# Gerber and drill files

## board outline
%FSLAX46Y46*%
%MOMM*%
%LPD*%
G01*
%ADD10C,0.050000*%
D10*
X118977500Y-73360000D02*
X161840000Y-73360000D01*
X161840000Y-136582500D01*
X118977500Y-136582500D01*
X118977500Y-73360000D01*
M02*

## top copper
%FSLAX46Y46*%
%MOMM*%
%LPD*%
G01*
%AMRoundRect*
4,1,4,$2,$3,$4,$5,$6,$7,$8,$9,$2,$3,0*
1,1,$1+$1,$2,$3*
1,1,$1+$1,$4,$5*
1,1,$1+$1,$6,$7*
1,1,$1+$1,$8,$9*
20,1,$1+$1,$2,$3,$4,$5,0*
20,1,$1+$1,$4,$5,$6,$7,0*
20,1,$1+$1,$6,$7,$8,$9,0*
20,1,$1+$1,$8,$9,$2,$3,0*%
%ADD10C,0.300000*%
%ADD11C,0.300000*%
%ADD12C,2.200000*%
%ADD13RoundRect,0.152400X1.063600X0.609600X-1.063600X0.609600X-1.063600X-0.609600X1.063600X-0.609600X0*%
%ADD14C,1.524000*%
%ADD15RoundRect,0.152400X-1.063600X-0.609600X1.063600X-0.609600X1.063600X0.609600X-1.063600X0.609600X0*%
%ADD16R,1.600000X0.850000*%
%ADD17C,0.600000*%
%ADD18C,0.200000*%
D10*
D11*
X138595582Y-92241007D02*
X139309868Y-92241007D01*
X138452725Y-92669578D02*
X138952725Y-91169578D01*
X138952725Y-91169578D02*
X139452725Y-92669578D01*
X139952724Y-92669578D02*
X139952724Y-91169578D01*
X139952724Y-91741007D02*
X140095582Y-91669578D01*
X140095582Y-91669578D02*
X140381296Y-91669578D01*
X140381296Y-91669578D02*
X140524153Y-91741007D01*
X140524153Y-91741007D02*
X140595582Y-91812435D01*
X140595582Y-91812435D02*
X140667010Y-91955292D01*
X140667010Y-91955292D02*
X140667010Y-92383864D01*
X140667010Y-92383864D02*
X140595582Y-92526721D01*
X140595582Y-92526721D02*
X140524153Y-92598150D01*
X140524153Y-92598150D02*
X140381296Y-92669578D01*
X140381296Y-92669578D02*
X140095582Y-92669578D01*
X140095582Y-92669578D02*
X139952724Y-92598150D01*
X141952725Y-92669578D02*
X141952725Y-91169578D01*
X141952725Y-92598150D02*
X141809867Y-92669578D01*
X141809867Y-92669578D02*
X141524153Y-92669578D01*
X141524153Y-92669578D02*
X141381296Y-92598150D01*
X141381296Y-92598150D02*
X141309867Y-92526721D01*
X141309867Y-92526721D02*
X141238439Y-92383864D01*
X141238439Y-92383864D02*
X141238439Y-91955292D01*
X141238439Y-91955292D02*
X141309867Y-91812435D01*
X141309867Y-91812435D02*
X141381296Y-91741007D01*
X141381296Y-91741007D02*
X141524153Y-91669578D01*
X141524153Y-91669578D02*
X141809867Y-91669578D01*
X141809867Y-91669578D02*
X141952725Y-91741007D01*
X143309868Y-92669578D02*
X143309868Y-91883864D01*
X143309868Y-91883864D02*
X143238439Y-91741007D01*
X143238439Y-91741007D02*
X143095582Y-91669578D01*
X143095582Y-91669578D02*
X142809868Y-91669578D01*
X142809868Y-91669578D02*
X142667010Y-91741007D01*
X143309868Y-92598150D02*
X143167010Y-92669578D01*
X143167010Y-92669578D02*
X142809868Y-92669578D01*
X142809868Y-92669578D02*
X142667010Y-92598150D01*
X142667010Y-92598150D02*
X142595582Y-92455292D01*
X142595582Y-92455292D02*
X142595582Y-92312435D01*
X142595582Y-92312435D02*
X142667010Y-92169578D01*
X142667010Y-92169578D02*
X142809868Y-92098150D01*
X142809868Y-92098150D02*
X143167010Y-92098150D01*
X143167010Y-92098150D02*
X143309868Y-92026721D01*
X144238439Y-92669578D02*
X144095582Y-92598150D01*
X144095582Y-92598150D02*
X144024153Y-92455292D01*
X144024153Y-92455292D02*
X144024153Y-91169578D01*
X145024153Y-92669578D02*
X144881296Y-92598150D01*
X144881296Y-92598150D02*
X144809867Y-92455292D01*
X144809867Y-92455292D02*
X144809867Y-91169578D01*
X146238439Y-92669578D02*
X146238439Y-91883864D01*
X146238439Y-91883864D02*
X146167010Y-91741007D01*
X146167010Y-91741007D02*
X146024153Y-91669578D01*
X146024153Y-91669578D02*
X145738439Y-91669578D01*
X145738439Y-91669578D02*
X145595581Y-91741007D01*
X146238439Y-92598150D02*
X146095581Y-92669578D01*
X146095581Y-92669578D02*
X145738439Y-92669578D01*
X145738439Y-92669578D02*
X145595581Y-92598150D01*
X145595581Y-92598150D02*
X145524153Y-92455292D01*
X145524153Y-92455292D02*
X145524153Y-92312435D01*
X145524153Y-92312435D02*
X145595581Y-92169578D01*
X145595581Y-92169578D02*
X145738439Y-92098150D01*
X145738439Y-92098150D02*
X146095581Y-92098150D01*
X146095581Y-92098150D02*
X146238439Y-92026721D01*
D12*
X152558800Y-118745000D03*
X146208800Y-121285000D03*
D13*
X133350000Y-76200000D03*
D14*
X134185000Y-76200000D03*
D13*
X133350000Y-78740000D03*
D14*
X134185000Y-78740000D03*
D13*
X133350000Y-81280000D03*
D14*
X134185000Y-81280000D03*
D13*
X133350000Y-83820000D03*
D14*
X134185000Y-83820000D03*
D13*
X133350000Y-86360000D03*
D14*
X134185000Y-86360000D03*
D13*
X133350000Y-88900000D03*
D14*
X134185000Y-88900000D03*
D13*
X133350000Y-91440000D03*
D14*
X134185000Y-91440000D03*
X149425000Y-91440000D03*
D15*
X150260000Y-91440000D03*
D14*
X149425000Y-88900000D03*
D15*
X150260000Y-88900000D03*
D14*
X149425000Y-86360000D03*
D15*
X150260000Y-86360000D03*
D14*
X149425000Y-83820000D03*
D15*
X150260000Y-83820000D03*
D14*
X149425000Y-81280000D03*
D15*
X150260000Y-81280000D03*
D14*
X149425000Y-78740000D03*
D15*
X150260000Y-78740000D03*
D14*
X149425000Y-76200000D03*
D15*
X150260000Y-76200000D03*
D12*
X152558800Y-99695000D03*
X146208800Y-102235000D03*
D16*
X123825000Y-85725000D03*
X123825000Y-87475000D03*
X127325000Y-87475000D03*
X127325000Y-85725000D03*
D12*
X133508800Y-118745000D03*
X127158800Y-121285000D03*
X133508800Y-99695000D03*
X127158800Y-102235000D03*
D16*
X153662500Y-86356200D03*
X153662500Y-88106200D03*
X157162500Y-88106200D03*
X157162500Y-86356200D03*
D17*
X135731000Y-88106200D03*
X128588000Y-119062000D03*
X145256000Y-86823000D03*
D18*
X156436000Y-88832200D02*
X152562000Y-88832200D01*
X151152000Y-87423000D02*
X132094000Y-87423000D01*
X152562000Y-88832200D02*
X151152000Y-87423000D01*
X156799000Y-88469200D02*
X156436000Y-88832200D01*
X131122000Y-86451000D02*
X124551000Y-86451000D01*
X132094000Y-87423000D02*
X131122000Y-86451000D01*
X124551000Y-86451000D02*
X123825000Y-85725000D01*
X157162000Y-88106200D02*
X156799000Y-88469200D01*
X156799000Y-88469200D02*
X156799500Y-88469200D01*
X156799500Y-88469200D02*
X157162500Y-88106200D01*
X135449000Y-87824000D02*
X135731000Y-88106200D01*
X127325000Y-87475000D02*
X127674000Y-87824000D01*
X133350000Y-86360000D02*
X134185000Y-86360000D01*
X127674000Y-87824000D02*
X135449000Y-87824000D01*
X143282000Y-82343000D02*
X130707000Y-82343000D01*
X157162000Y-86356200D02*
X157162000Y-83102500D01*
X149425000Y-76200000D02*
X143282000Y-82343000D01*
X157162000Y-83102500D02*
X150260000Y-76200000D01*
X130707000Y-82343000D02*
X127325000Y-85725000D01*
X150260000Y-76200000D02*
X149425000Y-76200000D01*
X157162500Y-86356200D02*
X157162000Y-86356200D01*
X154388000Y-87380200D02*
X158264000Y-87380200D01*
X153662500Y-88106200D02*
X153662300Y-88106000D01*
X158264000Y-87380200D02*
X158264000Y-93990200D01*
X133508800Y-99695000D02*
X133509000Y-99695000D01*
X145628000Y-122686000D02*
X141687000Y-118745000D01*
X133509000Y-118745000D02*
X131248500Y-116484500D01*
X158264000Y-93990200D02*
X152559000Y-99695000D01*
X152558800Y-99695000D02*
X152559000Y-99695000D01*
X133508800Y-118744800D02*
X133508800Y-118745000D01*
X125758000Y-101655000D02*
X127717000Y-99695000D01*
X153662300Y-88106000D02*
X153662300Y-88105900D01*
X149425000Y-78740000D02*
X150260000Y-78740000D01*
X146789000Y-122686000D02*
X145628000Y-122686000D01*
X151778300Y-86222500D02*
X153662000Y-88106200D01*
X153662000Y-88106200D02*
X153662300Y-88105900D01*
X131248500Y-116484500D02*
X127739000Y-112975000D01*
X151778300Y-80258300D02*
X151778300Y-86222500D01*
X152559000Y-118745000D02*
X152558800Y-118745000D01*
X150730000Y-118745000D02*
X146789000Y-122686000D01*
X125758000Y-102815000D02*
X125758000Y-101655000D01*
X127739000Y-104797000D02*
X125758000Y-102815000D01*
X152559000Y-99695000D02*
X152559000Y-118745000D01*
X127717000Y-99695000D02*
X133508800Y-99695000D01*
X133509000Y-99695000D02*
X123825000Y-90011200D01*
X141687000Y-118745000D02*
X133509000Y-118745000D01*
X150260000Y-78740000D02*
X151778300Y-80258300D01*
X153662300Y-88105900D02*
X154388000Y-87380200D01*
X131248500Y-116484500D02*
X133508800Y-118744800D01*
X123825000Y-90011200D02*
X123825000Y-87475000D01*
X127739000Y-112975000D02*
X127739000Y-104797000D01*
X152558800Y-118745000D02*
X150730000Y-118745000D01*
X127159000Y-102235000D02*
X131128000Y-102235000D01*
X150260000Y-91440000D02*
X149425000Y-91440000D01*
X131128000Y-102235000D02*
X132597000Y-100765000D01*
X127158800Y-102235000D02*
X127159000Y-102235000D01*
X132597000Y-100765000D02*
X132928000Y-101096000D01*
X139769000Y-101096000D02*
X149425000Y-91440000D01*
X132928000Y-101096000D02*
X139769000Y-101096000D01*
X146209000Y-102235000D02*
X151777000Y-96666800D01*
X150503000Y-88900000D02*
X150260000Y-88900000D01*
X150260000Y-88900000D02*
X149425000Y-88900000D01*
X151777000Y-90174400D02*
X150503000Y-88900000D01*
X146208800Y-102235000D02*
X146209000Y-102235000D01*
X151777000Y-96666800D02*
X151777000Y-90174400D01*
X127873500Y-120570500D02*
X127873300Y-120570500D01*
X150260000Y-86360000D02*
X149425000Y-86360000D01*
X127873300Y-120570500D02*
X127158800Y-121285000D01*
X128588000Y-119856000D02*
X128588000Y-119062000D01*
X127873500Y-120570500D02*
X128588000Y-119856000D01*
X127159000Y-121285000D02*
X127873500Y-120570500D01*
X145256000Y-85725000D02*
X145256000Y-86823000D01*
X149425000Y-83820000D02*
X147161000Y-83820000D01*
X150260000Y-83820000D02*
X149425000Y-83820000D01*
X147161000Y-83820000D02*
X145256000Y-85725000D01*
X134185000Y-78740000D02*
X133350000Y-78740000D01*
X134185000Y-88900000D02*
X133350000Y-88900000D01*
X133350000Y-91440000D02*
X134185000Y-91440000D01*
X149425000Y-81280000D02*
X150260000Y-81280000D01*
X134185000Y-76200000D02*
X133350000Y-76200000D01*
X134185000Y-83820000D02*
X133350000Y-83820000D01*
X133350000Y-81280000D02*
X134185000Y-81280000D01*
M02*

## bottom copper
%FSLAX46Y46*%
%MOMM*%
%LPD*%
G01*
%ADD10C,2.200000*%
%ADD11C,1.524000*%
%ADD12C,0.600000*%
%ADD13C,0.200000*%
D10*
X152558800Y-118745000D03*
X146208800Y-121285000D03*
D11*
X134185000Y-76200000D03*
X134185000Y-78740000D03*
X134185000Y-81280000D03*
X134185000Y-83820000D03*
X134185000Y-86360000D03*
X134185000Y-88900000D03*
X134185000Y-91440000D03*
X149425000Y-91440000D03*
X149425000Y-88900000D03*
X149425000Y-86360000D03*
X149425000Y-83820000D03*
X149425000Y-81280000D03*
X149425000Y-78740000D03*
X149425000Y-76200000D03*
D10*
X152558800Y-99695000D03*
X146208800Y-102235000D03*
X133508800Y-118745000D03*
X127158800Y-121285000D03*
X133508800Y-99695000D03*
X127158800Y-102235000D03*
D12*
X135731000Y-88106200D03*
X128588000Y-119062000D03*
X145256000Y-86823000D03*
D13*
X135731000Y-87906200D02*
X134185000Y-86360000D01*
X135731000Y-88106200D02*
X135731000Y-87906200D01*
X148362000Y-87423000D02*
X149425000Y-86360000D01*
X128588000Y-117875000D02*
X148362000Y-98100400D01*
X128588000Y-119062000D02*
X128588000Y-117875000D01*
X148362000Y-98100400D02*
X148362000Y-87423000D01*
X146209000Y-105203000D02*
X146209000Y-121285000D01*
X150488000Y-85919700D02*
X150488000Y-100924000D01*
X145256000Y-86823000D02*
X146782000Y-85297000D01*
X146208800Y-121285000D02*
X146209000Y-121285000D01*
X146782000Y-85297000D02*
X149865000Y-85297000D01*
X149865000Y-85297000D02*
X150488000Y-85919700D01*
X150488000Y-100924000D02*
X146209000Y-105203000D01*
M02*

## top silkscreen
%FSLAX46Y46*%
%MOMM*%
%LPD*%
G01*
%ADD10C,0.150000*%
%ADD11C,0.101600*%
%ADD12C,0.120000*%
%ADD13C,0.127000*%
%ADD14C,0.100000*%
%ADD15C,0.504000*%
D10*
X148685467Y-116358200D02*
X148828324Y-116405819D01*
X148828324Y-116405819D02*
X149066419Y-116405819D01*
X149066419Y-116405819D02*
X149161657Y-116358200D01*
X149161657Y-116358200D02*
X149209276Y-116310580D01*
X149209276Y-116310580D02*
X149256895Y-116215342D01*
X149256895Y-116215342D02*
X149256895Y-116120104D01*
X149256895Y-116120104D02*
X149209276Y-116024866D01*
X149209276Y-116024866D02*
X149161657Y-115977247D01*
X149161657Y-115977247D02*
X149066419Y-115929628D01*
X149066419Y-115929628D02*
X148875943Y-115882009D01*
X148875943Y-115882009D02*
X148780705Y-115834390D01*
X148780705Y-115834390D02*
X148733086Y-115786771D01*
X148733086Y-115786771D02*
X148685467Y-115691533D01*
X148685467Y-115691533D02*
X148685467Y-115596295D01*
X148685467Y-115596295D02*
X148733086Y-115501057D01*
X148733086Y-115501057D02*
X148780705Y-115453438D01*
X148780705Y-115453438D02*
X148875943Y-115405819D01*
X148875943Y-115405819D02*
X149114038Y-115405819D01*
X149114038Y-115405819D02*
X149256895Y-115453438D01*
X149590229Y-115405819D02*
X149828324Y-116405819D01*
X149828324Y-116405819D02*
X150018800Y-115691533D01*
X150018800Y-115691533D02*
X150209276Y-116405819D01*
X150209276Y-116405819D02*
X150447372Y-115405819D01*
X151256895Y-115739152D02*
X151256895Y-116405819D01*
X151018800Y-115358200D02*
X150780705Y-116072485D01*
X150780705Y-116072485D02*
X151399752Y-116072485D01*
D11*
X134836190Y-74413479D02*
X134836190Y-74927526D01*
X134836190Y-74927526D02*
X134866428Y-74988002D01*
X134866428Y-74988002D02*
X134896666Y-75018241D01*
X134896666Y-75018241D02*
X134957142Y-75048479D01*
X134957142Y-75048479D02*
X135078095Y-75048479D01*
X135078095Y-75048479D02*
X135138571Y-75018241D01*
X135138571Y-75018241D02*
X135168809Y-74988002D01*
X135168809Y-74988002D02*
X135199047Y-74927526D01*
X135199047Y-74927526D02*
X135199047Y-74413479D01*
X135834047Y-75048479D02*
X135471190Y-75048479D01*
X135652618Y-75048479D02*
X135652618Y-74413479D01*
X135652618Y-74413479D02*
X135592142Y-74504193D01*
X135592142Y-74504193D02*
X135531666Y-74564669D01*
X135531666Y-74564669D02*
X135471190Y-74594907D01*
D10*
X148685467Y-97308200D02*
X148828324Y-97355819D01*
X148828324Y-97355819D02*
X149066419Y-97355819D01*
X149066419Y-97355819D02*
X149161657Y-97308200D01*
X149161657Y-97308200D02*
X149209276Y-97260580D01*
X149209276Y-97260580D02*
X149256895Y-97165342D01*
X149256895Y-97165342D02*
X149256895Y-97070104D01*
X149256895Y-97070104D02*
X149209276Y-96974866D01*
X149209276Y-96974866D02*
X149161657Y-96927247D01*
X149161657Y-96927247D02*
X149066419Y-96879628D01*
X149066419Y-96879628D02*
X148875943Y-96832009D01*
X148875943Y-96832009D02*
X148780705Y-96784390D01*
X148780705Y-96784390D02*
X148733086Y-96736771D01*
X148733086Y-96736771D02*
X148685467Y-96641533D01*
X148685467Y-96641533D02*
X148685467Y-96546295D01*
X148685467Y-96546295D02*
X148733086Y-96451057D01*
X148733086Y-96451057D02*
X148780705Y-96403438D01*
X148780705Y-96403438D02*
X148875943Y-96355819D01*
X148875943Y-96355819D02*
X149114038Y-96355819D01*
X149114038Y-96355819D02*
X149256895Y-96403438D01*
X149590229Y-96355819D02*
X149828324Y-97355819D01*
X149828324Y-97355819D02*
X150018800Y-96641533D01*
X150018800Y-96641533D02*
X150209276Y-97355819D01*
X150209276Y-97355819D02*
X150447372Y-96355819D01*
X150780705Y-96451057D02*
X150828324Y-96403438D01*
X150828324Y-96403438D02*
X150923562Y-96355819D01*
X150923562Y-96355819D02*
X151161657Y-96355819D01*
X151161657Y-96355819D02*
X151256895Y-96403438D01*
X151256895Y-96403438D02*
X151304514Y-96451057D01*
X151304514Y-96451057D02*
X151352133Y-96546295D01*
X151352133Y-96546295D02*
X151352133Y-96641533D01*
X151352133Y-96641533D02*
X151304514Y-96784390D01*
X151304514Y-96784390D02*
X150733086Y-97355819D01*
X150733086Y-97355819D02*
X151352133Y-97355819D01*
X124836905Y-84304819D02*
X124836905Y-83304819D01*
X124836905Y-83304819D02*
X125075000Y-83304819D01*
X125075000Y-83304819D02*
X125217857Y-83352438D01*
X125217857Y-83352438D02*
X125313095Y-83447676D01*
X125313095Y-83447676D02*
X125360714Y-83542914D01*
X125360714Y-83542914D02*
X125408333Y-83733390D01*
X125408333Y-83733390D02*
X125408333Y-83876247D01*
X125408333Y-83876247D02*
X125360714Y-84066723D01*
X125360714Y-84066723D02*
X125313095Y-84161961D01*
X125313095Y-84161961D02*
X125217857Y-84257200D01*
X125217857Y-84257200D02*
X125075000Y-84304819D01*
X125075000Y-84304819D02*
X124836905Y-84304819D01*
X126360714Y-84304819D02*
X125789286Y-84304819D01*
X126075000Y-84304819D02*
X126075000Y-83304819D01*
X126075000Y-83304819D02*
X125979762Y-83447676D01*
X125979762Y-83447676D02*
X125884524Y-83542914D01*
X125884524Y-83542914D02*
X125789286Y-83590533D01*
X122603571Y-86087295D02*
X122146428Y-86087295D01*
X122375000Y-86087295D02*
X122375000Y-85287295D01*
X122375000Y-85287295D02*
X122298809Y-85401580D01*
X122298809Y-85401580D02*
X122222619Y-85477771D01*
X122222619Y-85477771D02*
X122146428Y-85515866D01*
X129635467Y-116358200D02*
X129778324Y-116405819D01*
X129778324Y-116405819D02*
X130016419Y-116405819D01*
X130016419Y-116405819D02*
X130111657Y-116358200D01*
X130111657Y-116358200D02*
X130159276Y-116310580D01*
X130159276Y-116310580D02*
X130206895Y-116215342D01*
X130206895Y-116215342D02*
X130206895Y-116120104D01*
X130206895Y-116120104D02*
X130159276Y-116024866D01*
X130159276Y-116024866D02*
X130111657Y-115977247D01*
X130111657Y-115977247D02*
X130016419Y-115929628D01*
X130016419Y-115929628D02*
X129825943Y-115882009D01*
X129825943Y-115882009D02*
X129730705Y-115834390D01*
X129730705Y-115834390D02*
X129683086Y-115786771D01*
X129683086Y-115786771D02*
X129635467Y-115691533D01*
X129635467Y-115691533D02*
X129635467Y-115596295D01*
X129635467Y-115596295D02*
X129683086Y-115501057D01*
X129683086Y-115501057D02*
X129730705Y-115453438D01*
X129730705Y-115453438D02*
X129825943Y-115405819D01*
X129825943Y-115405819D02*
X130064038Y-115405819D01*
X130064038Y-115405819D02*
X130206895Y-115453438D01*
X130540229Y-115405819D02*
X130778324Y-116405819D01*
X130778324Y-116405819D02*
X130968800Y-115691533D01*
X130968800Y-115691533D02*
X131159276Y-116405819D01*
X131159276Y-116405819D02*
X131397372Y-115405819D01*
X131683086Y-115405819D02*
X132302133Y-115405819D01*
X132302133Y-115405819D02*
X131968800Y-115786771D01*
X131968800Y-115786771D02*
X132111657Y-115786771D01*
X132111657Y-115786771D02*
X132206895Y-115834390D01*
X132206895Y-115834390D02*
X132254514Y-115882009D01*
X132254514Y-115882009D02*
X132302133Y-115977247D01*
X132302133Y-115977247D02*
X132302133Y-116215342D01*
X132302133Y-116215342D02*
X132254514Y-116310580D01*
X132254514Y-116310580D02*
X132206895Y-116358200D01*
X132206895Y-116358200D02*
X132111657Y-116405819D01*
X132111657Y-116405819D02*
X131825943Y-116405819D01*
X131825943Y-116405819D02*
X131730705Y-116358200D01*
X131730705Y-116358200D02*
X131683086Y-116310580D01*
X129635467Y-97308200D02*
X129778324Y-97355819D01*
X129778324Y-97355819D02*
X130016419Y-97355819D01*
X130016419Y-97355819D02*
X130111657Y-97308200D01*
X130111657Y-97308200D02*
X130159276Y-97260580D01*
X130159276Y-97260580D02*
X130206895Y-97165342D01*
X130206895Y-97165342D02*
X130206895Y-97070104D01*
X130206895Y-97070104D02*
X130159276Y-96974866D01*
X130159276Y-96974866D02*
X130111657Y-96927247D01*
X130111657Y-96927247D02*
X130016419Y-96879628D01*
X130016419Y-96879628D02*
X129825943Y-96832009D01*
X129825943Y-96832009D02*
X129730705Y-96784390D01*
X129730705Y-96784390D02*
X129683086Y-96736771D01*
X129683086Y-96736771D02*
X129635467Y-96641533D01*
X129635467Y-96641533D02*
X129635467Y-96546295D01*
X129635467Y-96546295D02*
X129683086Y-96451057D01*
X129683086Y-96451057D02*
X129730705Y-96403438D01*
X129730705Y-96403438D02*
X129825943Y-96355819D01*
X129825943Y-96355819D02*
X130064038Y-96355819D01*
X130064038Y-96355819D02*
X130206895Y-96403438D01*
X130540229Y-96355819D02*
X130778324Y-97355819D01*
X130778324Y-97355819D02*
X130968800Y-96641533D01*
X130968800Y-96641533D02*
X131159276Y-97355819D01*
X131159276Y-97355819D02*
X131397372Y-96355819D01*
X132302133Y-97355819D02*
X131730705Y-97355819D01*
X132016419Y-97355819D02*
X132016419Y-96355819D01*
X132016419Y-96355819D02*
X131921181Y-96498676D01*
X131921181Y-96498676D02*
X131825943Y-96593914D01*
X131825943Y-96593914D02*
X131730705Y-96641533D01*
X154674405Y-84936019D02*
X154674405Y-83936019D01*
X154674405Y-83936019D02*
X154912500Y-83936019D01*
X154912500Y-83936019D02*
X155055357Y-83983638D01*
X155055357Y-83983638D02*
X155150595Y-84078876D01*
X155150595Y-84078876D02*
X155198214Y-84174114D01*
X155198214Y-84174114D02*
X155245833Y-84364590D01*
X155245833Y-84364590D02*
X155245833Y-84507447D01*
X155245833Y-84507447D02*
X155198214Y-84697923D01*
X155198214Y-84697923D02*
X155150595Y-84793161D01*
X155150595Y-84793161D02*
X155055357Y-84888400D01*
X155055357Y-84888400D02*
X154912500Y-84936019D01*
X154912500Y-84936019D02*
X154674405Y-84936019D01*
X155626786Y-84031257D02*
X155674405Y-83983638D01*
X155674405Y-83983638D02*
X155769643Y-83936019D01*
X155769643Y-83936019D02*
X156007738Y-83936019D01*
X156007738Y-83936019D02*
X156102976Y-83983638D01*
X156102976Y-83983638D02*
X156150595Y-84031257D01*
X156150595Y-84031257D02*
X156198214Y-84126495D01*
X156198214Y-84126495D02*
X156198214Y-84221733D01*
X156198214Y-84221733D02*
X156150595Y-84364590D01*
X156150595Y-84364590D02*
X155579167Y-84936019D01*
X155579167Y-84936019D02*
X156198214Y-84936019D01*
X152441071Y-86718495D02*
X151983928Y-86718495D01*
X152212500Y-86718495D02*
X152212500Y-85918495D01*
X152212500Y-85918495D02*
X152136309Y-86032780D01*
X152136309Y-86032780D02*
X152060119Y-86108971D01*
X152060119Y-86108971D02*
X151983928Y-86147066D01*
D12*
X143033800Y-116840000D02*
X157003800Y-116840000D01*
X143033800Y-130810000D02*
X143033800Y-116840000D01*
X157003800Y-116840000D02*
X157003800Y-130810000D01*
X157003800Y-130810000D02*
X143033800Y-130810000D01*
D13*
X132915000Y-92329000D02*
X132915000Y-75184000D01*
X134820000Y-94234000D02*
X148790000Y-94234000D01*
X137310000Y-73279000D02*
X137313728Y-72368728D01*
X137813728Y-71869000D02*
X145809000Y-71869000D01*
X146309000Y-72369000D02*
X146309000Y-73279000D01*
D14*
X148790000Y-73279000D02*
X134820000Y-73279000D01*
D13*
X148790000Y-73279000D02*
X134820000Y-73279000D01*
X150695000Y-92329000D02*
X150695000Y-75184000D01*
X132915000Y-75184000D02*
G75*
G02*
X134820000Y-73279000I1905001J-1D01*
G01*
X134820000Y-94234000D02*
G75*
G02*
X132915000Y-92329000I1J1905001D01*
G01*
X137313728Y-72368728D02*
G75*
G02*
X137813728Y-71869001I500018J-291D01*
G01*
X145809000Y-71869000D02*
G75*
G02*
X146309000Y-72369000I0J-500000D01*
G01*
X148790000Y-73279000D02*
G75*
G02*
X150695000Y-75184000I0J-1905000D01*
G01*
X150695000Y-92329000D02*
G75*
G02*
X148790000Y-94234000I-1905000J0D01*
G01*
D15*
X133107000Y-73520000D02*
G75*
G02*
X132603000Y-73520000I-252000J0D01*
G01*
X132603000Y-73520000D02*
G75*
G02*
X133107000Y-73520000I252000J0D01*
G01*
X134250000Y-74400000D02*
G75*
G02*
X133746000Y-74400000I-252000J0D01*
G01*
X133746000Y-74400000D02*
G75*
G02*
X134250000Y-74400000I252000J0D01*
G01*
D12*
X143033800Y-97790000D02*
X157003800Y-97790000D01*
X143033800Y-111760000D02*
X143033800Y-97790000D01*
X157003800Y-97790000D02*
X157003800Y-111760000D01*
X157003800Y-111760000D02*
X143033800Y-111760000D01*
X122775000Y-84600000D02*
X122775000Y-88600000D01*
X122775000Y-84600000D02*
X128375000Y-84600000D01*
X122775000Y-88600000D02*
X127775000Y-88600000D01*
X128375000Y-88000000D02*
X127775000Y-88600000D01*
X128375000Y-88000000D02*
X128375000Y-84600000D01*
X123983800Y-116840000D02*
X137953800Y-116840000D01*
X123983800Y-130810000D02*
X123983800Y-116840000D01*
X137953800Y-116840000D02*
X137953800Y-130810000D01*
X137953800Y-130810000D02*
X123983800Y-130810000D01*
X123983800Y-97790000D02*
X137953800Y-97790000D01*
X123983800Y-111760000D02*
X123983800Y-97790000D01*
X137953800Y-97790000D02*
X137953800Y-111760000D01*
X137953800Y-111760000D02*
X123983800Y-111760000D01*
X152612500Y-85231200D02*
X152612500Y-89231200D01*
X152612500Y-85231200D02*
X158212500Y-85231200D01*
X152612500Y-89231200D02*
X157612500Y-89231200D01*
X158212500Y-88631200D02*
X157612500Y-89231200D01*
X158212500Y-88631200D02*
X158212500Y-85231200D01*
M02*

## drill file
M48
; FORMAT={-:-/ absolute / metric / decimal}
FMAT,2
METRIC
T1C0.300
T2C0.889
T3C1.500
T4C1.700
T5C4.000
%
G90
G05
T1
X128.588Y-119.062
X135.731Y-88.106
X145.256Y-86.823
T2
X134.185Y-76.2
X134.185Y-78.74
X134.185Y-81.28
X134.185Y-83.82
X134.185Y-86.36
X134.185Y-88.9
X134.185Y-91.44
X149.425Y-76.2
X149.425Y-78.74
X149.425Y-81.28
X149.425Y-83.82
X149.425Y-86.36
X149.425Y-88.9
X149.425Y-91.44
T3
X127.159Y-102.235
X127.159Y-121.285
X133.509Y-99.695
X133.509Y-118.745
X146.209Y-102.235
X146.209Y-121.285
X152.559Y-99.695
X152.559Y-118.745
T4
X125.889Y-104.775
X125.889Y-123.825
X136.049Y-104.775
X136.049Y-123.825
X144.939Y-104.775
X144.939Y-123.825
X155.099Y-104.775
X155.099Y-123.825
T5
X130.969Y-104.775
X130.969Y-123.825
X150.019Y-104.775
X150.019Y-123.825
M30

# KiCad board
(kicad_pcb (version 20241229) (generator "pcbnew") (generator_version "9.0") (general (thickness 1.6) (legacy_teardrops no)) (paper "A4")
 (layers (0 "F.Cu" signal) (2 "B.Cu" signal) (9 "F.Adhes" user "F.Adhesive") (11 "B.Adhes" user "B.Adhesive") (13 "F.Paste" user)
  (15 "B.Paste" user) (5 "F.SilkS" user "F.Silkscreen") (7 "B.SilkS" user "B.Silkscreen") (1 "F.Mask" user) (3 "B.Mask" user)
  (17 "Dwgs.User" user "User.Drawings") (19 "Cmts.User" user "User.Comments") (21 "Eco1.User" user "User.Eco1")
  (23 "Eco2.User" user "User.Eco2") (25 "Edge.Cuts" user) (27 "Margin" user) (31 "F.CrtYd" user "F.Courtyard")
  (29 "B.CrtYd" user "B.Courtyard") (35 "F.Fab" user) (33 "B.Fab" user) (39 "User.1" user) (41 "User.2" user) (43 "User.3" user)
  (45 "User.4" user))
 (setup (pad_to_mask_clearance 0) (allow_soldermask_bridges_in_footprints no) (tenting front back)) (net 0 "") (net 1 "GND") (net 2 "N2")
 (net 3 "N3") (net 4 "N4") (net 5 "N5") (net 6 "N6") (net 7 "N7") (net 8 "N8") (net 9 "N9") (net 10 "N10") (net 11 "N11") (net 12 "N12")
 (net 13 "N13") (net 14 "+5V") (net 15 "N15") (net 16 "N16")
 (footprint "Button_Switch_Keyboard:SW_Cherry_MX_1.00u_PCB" (layer "F.Cu") (at 152.5588 118.745)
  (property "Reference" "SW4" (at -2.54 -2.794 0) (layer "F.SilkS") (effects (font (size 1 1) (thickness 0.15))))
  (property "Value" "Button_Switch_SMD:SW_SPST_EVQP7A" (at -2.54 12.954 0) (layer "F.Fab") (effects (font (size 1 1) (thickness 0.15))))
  (fp_line (start -9.525 -1.905) (end 4.445 -1.905) (stroke (width 0.12) (type solid)) (layer "F.SilkS"))
  (fp_line (start -9.525 12.065) (end -9.525 -1.905) (stroke (width 0.12) (type solid)) (layer "F.SilkS"))
  (fp_line (start 4.445 -1.905) (end 4.445 12.065) (stroke (width 0.12) (type solid)) (layer "F.SilkS"))
  (fp_line (start 4.445 12.065) (end -9.525 12.065) (stroke (width 0.12) (type solid)) (layer "F.SilkS"))
  (pad "" np_thru_hole circle (at -7.62 5.08) (size 1.7 1.7) (drill 1.7) (layers "*.Cu" "*.Mask"))
  (pad "" np_thru_hole circle (at -2.54 5.08) (size 4 4) (drill 4) (layers "*.Cu" "*.Mask"))
  (pad "" np_thru_hole circle (at 2.54 5.08) (size 1.7 1.7) (drill 1.7) (layers "*.Cu" "*.Mask"))
  (pad "1" thru_hole circle (at 0 0) (size 2.2 2.2) (drill 1.5) (layers "*.Cu" "*.Mask") (remove_unused_layers no) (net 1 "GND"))
  (pad "2" thru_hole circle (at -6.35 2.54) (size 2.2 2.2) (drill 1.5) (layers "*.Cu" "*.Mask") (remove_unused_layers no) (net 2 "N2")))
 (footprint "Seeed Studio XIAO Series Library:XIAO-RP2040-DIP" (layer "F.Cu") (at 141.805 83.82)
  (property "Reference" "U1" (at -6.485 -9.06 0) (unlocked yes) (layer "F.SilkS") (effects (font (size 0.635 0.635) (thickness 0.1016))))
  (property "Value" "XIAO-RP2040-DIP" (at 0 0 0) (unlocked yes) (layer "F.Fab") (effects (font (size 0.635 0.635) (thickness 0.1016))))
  (fp_line (start -8.89 8.509) (end -8.89 -8.636) (stroke (width 0.127) (type solid)) (layer "F.SilkS"))
  (fp_line (start -6.985 10.414) (end 6.985 10.414) (stroke (width 0.127) (type solid)) (layer "F.SilkS"))
  (fp_line (start -4.495 -10.541) (end -4.491272 -11.451272) (stroke (width 0.127) (type solid)) (layer "F.SilkS"))
  (fp_line (start -3.991272 -11.951) (end 4.004 -11.951) (stroke (width 0.127) (type solid)) (layer "F.SilkS"))
  (fp_line (start 4.504 -11.451) (end 4.504 -10.541) (stroke (width 0.127) (type solid)) (layer "F.SilkS"))
  (fp_line (start 6.985 -10.541) (end -6.985 -10.541) (stroke (width 0.1) (type solid)) (layer "F.SilkS"))
  (fp_line (start 6.985 -10.541) (end -6.985 -10.541) (stroke (width 0.127) (type solid)) (layer "F.SilkS"))
  (fp_line (start 8.89 8.509) (end 8.89 -8.636) (stroke (width 0.127) (type solid)) (layer "F.SilkS"))
  (fp_arc (start -8.89 -8.636) (mid -8.332038 -9.983038) (end -6.985 -10.541) (stroke (width 0.127) (type solid)) (layer "F.SilkS"))
  (fp_arc (start -6.985 10.414) (mid -8.332038 9.856038) (end -8.89 8.509) (stroke (width 0.127) (type solid)) (layer "F.SilkS"))
  (fp_arc (start -4.491272 -11.451272) (mid -4.344728 -11.80464) (end -3.991272 -11.951) (stroke (width 0.127) (type default))
   (layer "F.SilkS"))
  (fp_arc (start 4.004 -11.951) (mid 4.357553 -11.804553) (end 4.504 -11.451) (stroke (width 0.127) (type default)) (layer "F.SilkS"))
  (fp_arc (start 6.985 -10.541) (mid 8.332038 -9.983038) (end 8.89 -8.636) (stroke (width 0.127) (type solid)) (layer "F.SilkS"))
  (fp_arc (start 8.89 8.509) (mid 8.332038 9.856038) (end 6.985 10.414) (stroke (width 0.127) (type solid)) (layer "F.SilkS"))
  (fp_circle (center -8.95 -10.3) (end -8.95 -10.554) (stroke (width 0.5) (type solid)) (fill yes) (layer "F.SilkS"))
  (fp_circle (center -7.807 -9.42) (end -7.807 -9.674) (stroke (width 0.5) (type solid)) (fill yes) (layer "F.SilkS"))
  (pad "1" smd roundrect (at -8.455 -7.62 180) (size 2.432 1.524) (layers "F.Cu" "F.Mask") (roundrect_rratio 0.1) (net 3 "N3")
   (thermal_bridge_angle 45))
  (pad "1" thru_hole circle (at -7.62 -7.62 180) (size 1.524 1.524) (drill 0.889) (layers "*.Cu" "*.Mask") (remove_unused_layers no)
   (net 3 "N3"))
  (pad "2" smd roundrect (at -8.455 -5.08 180) (size 2.432 1.524) (layers "F.Cu" "F.Mask") (roundrect_rratio 0.1) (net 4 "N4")
   (thermal_bridge_angle 45))
  (pad "2" thru_hole circle (at -7.62 -5.08 180) (size 1.524 1.524) (drill 0.889) (layers "*.Cu" "*.Mask") (remove_unused_layers no)
   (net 4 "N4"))
  (pad "3" smd roundrect (at -8.455 -2.54 180) (size 2.432 1.524) (layers "F.Cu" "F.Mask") (roundrect_rratio 0.1) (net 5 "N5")
   (thermal_bridge_angle 45))
  (pad "3" thru_hole circle (at -7.62 -2.54 180) (size 1.524 1.524) (drill 0.889) (layers "*.Cu" "*.Mask") (remove_unused_layers no)
   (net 5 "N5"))
  (pad "4" smd roundrect (at -8.455 0 180) (size 2.432 1.524) (layers "F.Cu" "F.Mask") (roundrect_rratio 0.1) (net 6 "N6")
   (thermal_bridge_angle 45))
  (pad "4" thru_hole circle (at -7.62 0 180) (size 1.524 1.524) (drill 0.889) (layers "*.Cu" "*.Mask") (remove_unused_layers no)
   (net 6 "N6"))
  (pad "5" smd roundrect (at -8.455 2.54 180) (size 2.432 1.524) (layers "F.Cu" "F.Mask") (roundrect_rratio 0.1) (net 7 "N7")
   (thermal_bridge_angle 45))
  (pad "5" thru_hole circle (at -7.62 2.54 180) (size 1.524 1.524) (drill 0.889) (layers "*.Cu" "*.Mask") (remove_unused_layers no)
   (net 7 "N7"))
  (pad "6" smd roundrect (at -8.455 5.08 180) (size 2.432 1.524) (layers "F.Cu" "F.Mask") (roundrect_rratio 0.1) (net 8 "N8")
   (thermal_bridge_angle 45))
  (pad "6" thru_hole circle (at -7.62 5.08 180) (size 1.524 1.524) (drill 0.889) (layers "*.Cu" "*.Mask") (remove_unused_layers no)
   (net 8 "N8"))
  (pad "7" smd roundrect (at -8.455 7.62 180) (size 2.432 1.524) (layers "F.Cu" "F.Mask") (roundrect_rratio 0.1) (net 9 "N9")
   (thermal_bridge_angle 45))
  (pad "7" thru_hole circle (at -7.62 7.62 180) (size 1.524 1.524) (drill 0.889) (layers "*.Cu" "*.Mask") (remove_unused_layers no)
   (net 9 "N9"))
  (pad "8" thru_hole circle (at 7.62 7.62) (size 1.524 1.524) (drill 0.889) (layers "*.Cu" "*.Mask") (remove_unused_layers no)
   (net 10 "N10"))
  (pad "8" smd roundrect (at 8.455 7.62) (size 2.432 1.524) (layers "F.Cu" "F.Mask") (roundrect_rratio 0.1) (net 10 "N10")
   (thermal_bridge_angle 45))
  (pad "9" thru_hole circle (at 7.62 5.08) (size 1.524 1.524) (drill 0.889) (layers "*.Cu" "*.Mask") (remove_unused_layers no)
   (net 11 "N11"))
  (pad "9" smd roundrect (at 8.455 5.08) (size 2.432 1.524) (layers "F.Cu" "F.Mask") (roundrect_rratio 0.1) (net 11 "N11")
   (thermal_bridge_angle 45))
  (pad "10" thru_hole circle (at 7.62 2.54) (size 1.524 1.524) (drill 0.889) (layers "*.Cu" "*.Mask") (remove_unused_layers no)
   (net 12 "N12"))
  (pad "10" smd roundrect (at 8.455 2.54) (size 2.432 1.524) (layers "F.Cu" "F.Mask") (roundrect_rratio 0.1) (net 12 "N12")
   (thermal_bridge_angle 45))
  (pad "11" thru_hole circle (at 7.62 0) (size 1.524 1.524) (drill 0.889) (layers "*.Cu" "*.Mask") (remove_unused_layers no) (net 2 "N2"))
  (pad "11" smd roundrect (at 8.455 0) (size 2.432 1.524) (layers "F.Cu" "F.Mask") (roundrect_rratio 0.1) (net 2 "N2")
   (thermal_bridge_angle 45))
  (pad "12" thru_hole circle (at 7.62 -2.54) (size 1.524 1.524) (drill 0.889) (layers "*.Cu" "*.Mask") (remove_unused_layers no)
   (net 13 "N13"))
  (pad "12" smd roundrect (at 8.455 -2.54) (size 2.432 1.524) (layers "F.Cu" "F.Mask") (roundrect_rratio 0.1) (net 13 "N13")
   (thermal_bridge_angle 45))
  (pad "13" thru_hole circle (at 7.62 -5.08) (size 1.524 1.524) (drill 0.889) (layers "*.Cu" "*.Mask") (remove_unused_layers no)
   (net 1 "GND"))
  (pad "13" smd roundrect (at 8.455 -5.08) (size 2.432 1.524) (layers "F.Cu" "F.Mask") (roundrect_rratio 0.1) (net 1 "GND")
   (thermal_bridge_angle 45))
  (pad "14" thru_hole circle (at 7.62 -7.62) (size 1.524 1.524) (drill 0.889) (layers "*.Cu" "*.Mask") (remove_unused_layers no)
   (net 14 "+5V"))
  (pad "14" smd roundrect (at 8.455 -7.62) (size 2.432 1.524) (layers "F.Cu" "F.Mask") (roundrect_rratio 0.1) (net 14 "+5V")
   (thermal_bridge_angle 45)))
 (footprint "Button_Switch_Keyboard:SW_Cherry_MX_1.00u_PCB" (layer "F.Cu") (at 152.5588 99.695)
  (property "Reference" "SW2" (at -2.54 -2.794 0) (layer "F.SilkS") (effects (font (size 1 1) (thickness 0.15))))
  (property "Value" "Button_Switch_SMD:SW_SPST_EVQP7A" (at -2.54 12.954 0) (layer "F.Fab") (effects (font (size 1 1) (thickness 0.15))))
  (fp_line (start -9.525 -1.905) (end 4.445 -1.905) (stroke (width 0.12) (type solid)) (layer "F.SilkS"))
  (fp_line (start -9.525 12.065) (end -9.525 -1.905) (stroke (width 0.12) (type solid)) (layer "F.SilkS"))
  (fp_line (start 4.445 -1.905) (end 4.445 12.065) (stroke (width 0.12) (type solid)) (layer "F.SilkS"))
  (fp_line (start 4.445 12.065) (end -9.525 12.065) (stroke (width 0.12) (type solid)) (layer "F.SilkS"))
  (pad "" np_thru_hole circle (at -7.62 5.08) (size 1.7 1.7) (drill 1.7) (layers "*.Cu" "*.Mask"))
  (pad "" np_thru_hole circle (at -2.54 5.08) (size 4 4) (drill 4) (layers "*.Cu" "*.Mask"))
  (pad "" np_thru_hole circle (at 2.54 5.08) (size 1.7 1.7) (drill 1.7) (layers "*.Cu" "*.Mask"))
  (pad "1" thru_hole circle (at 0 0) (size 2.2 2.2) (drill 1.5) (layers "*.Cu" "*.Mask") (remove_unused_layers no) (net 1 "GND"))
  (pad "2" thru_hole circle (at -6.35 2.54) (size 2.2 2.2) (drill 1.5) (layers "*.Cu" "*.Mask") (remove_unused_layers no) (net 11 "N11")))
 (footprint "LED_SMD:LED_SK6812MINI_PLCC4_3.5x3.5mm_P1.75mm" (layer "F.Cu") (at 125.575 86.6)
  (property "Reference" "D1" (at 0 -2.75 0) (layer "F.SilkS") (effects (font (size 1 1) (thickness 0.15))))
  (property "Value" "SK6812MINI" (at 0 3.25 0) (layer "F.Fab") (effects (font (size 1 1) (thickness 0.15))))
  (fp_line (start -2.8 -2) (end -2.8 2) (stroke (width 0.12) (type default)) (layer "F.SilkS"))
  (fp_line (start -2.8 -2) (end 2.8 -2) (stroke (width 0.12) (type solid)) (layer "F.SilkS"))
  (fp_line (start -2.8 2) (end 2.2 2) (stroke (width 0.12) (type solid)) (layer "F.SilkS"))
  (fp_line (start 2.8 1.4) (end 2.2 2) (stroke (width 0.12) (type default)) (layer "F.SilkS"))
  (fp_line (start 2.8 1.4) (end 2.8 -2) (stroke (width 0.12) (type solid)) (layer "F.SilkS"))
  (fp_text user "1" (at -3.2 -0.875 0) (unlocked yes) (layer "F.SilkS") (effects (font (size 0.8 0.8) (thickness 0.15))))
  (pad "1" smd rect (at -1.75 -0.875) (size 1.6 0.85) (layers "F.Cu" "F.Mask" "F.Paste") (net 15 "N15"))
  (pad "2" smd rect (at -1.75 0.875) (size 1.6 0.85) (layers "F.Cu" "F.Mask" "F.Paste") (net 1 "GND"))
  (pad "3" smd rect (at 1.75 0.875) (size 1.6 0.85) (layers "F.Cu" "F.Mask" "F.Paste") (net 7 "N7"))
  (pad "4" smd rect (at 1.75 -0.875) (size 1.6 0.85) (layers "F.Cu" "F.Mask" "F.Paste") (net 14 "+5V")))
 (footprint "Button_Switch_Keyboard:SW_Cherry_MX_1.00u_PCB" (layer "F.Cu") (at 133.5088 118.745)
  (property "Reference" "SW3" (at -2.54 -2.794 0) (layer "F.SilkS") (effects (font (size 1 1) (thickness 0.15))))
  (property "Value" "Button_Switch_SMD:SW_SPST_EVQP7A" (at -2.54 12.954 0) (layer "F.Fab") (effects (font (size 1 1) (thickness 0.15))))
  (fp_line (start -9.525 -1.905) (end 4.445 -1.905) (stroke (width 0.12) (type solid)) (layer "F.SilkS"))
  (fp_line (start -9.525 12.065) (end -9.525 -1.905) (stroke (width 0.12) (type solid)) (layer "F.SilkS"))
  (fp_line (start 4.445 -1.905) (end 4.445 12.065) (stroke (width 0.12) (type solid)) (layer "F.SilkS"))
  (fp_line (start 4.445 12.065) (end -9.525 12.065) (stroke (width 0.12) (type solid)) (layer "F.SilkS"))
  (pad "" np_thru_hole circle (at -7.62 5.08) (size 1.7 1.7) (drill 1.7) (layers "*.Cu" "*.Mask"))
  (pad "" np_thru_hole circle (at -2.54 5.08) (size 4 4) (drill 4) (layers "*.Cu" "*.Mask"))
  (pad "" np_thru_hole circle (at 2.54 5.08) (size 1.7 1.7) (drill 1.7) (layers "*.Cu" "*.Mask"))
  (pad "1" thru_hole circle (at 0 0) (size 2.2 2.2) (drill 1.5) (layers "*.Cu" "*.Mask") (remove_unused_layers no) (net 1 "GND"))
  (pad "2" thru_hole circle (at -6.35 2.54) (size 2.2 2.2) (drill 1.5) (layers "*.Cu" "*.Mask") (remove_unused_layers no) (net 12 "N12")))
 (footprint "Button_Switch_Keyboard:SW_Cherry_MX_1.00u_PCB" (layer "F.Cu") (at 133.5088 99.695)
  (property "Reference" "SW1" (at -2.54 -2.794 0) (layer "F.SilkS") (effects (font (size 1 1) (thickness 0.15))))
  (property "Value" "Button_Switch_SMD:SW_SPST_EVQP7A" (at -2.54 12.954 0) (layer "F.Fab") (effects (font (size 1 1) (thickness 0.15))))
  (fp_line (start -9.525 -1.905) (end 4.445 -1.905) (stroke (width 0.12) (type solid)) (layer "F.SilkS"))
  (fp_line (start -9.525 12.065) (end -9.525 -1.905) (stroke (width 0.12) (type solid)) (layer "F.SilkS"))
  (fp_line (start 4.445 -1.905) (end 4.445 12.065) (stroke (width 0.12) (type solid)) (layer "F.SilkS"))
  (fp_line (start 4.445 12.065) (end -9.525 12.065) (stroke (width 0.12) (type solid)) (layer "F.SilkS"))
  (pad "" np_thru_hole circle (at -7.62 5.08) (size 1.7 1.7) (drill 1.7) (layers "*.Cu" "*.Mask"))
  (pad "" np_thru_hole circle (at -2.54 5.08) (size 4 4) (drill 4) (layers "*.Cu" "*.Mask"))
  (pad "" np_thru_hole circle (at 2.54 5.08) (size 1.7 1.7) (drill 1.7) (layers "*.Cu" "*.Mask"))
  (pad "1" thru_hole circle (at 0 0) (size 2.2 2.2) (drill 1.5) (layers "*.Cu" "*.Mask") (remove_unused_layers no) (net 1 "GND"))
  (pad "2" thru_hole circle (at -6.35 2.54) (size 2.2 2.2) (drill 1.5) (layers "*.Cu" "*.Mask") (remove_unused_layers no) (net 10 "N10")))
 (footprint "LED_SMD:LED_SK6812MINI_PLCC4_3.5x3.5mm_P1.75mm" (layer "F.Cu") (at 155.4125 87.2312)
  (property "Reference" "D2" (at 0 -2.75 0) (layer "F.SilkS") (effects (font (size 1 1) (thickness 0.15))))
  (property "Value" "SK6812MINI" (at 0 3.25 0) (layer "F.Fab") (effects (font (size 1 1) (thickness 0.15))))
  (fp_line (start -2.8 -2) (end -2.8 2) (stroke (width 0.12) (type default)) (layer "F.SilkS"))
  (fp_line (start -2.8 -2) (end 2.8 -2) (stroke (width 0.12) (type solid)) (layer "F.SilkS"))
  (fp_line (start -2.8 2) (end 2.2 2) (stroke (width 0.12) (type solid)) (layer "F.SilkS"))
  (fp_line (start 2.8 1.4) (end 2.2 2) (stroke (width 0.12) (type default)) (layer "F.SilkS"))
  (fp_line (start 2.8 1.4) (end 2.8 -2) (stroke (width 0.12) (type solid)) (layer "F.SilkS"))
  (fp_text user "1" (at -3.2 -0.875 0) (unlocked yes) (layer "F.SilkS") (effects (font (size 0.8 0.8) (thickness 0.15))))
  (pad "1" smd rect (at -1.75 -0.875) (size 1.6 0.85) (layers "F.Cu" "F.Mask" "F.Paste") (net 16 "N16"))
  (pad "2" smd rect (at -1.75 0.875) (size 1.6 0.85) (layers "F.Cu" "F.Mask" "F.Paste") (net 1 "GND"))
  (pad "3" smd rect (at 1.75 0.875) (size 1.6 0.85) (layers "F.Cu" "F.Mask" "F.Paste") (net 15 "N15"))
  (pad "4" smd rect (at 1.75 -0.875) (size 1.6 0.85) (layers "F.Cu" "F.Mask" "F.Paste") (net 14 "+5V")))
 (gr_rect (start 118.9775 73.36) (end 161.84 136.5825) (stroke (width 0.05) (type solid)) (fill no) (layer "Edge.Cuts"))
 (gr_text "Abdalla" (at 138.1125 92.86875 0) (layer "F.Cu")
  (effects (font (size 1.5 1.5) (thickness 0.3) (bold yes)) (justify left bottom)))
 (segment (start 156.436 88.8322) (end 152.562 88.8322) (width 0.2) (layer "F.Cu") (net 15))
 (segment (start 151.152 87.423) (end 132.094 87.423) (width 0.2) (layer "F.Cu") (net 15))
 (segment (start 152.562 88.8322) (end 151.152 87.423) (width 0.2) (layer "F.Cu") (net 15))
 (segment (start 156.799 88.4692) (end 156.436 88.8322) (width 0.2) (layer "F.Cu") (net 15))
 (segment (start 131.122 86.451) (end 124.551 86.451) (width 0.2) (layer "F.Cu") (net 15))
 (segment (start 132.094 87.423) (end 131.122 86.451) (width 0.2) (layer "F.Cu") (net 15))
 (segment (start 124.551 86.451) (end 123.825 85.725) (width 0.2) (layer "F.Cu") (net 15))
 (segment (start 157.162 88.1062) (end 156.799 88.4692) (width 0.2) (layer "F.Cu") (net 15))
 (segment (start 156.799 88.4692) (end 156.7995 88.4692) (width 0.2) (layer "F.Cu") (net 15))
 (segment (start 156.7995 88.4692) (end 157.1625 88.1062) (width 0.2) (layer "F.Cu") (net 15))
 (segment (start 135.449 87.824) (end 135.731 88.1062) (width 0.2) (layer "F.Cu") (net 7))
 (segment (start 127.325 87.475) (end 127.674 87.824) (width 0.2) (layer "F.Cu") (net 7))
 (segment (start 133.35 86.36) (end 134.185 86.36) (width 0.2) (layer "F.Cu") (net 7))
 (segment (start 127.674 87.824) (end 135.449 87.824) (width 0.2) (layer "F.Cu") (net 7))
 (via (at 135.731 88.1062) (size 0.6) (drill 0.3) (layers "F.Cu" "B.Cu") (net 7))
 (segment (start 135.731 87.9062) (end 134.185 86.36) (width 0.2) (layer "B.Cu") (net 7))
 (segment (start 135.731 88.1062) (end 135.731 87.9062) (width 0.2) (layer "B.Cu") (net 7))
 (segment (start 143.282 82.343) (end 130.707 82.343) (width 0.2) (layer "F.Cu") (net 14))
 (segment (start 157.162 86.3562) (end 157.162 83.1025) (width 0.2) (layer "F.Cu") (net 14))
 (segment (start 149.425 76.2) (end 143.282 82.343) (width 0.2) (layer "F.Cu") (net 14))
 (segment (start 157.162 83.1025) (end 150.26 76.2) (width 0.2) (layer "F.Cu") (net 14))
 (segment (start 130.707 82.343) (end 127.325 85.725) (width 0.2) (layer "F.Cu") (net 14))
 (segment (start 150.26 76.2) (end 149.425 76.2) (width 0.2) (layer "F.Cu") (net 14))
 (segment (start 157.1625 86.3562) (end 157.162 86.3562) (width 0.2) (layer "F.Cu") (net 14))
 (segment (start 154.388 87.3802) (end 158.264 87.3802) (width 0.2) (layer "F.Cu") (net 1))
 (segment (start 153.6625 88.1062) (end 153.6623 88.106) (width 0.2) (layer "F.Cu") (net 1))
 (segment (start 158.264 87.3802) (end 158.264 93.9902) (width 0.2) (layer "F.Cu") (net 1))
 (segment (start 133.5088 99.695) (end 133.509 99.695) (width 0.2) (layer "F.Cu") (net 1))
 (segment (start 145.628 122.686) (end 141.687 118.745) (width 0.2) (layer "F.Cu") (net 1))
 (segment (start 133.509 118.745) (end 131.2485 116.4845) (width 0.2) (layer "F.Cu") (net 1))
 (segment (start 158.264 93.9902) (end 152.559 99.695) (width 0.2) (layer "F.Cu") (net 1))
 (segment (start 152.5588 99.695) (end 152.559 99.695) (width 0.2) (layer "F.Cu") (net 1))
 (segment (start 133.5088 118.7448) (end 133.5088 118.745) (width 0.2) (layer "F.Cu") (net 1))
 (segment (start 125.758 101.655) (end 127.717 99.695) (width 0.2) (layer "F.Cu") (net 1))
 (segment (start 153.6623 88.106) (end 153.6623 88.1059) (width 0.2) (layer "F.Cu") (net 1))
 (segment (start 149.425 78.74) (end 150.26 78.74) (width 0.2) (layer "F.Cu") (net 1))
 (segment (start 146.789 122.686) (end 145.628 122.686) (width 0.2) (layer "F.Cu") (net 1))
 (segment (start 151.7783 86.2225) (end 153.662 88.1062) (width 0.2) (layer "F.Cu") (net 1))
 (segment (start 153.662 88.1062) (end 153.6623 88.1059) (width 0.2) (layer "F.Cu") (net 1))
 (segment (start 131.2485 116.4845) (end 127.739 112.975) (width 0.2) (layer "F.Cu") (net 1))
 (segment (start 151.7783 80.2583) (end 151.7783 86.2225) (width 0.2) (layer "F.Cu") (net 1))
 (segment (start 152.559 118.745) (end 152.5588 118.745) (width 0.2) (layer "F.Cu") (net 1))
 (segment (start 150.73 118.745) (end 146.789 122.686) (width 0.2) (layer "F.Cu") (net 1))
 (segment (start 125.758 102.815) (end 125.758 101.655) (width 0.2) (layer "F.Cu") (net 1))
 (segment (start 127.739 104.797) (end 125.758 102.815) (width 0.2) (layer "F.Cu") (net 1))
 (segment (start 152.559 99.695) (end 152.559 118.745) (width 0.2) (layer "F.Cu") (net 1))
 (segment (start 127.717 99.695) (end 133.5088 99.695) (width 0.2) (layer "F.Cu") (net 1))
 (segment (start 133.509 99.695) (end 123.825 90.0112) (width 0.2) (layer "F.Cu") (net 1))
 (segment (start 141.687 118.745) (end 133.509 118.745) (width 0.2) (layer "F.Cu") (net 1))
 (segment (start 150.26 78.74) (end 151.7783 80.2583) (width 0.2) (layer "F.Cu") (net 1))
 (segment (start 153.6623 88.1059) (end 154.388 87.3802) (width 0.2) (layer "F.Cu") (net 1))
 (segment (start 131.2485 116.4845) (end 133.5088 118.7448) (width 0.2) (layer "F.Cu") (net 1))
 (segment (start 123.825 90.0112) (end 123.825 87.475) (width 0.2) (layer "F.Cu") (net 1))
 (segment (start 127.739 112.975) (end 127.739 104.797) (width 0.2) (layer "F.Cu") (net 1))
 (segment (start 152.5588 118.745) (end 150.73 118.745) (width 0.2) (layer "F.Cu") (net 1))
 (segment (start 127.159 102.235) (end 131.128 102.235) (width 0.2) (layer "F.Cu") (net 10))
 (segment (start 150.26 91.44) (end 149.425 91.44) (width 0.2) (layer "F.Cu") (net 10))
 (segment (start 131.128 102.235) (end 132.597 100.765) (width 0.2) (layer "F.Cu") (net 10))
 (segment (start 127.1588 102.235) (end 127.159 102.235) (width 0.2) (layer "F.Cu") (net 10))
 (segment (start 132.597 100.765) (end 132.928 101.096) (width 0.2) (layer "F.Cu") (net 10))
 (segment (start 139.769 101.096) (end 149.425 91.44) (width 0.2) (layer "F.Cu") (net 10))
 (segment (start 132.928 101.096) (end 139.769 101.096) (width 0.2) (layer "F.Cu") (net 10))
 (segment (start 146.209 102.235) (end 151.777 96.6668) (width 0.2) (layer "F.Cu") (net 11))
 (segment (start 150.503 88.9) (end 150.26 88.9) (width 0.2) (layer "F.Cu") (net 11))
 (segment (start 150.26 88.9) (end 149.425 88.9) (width 0.2) (layer "F.Cu") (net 11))
 (segment (start 151.777 90.1744) (end 150.503 88.9) (width 0.2) (layer "F.Cu") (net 11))
 (segment (start 146.2088 102.235) (end 146.209 102.235) (width 0.2) (layer "F.Cu") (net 11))
 (segment (start 151.777 96.6668) (end 151.777 90.1744) (width 0.2) (layer "F.Cu") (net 11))
 (segment (start 127.8735 120.5705) (end 127.8733 120.5705) (width 0.2) (layer "F.Cu") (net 12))
 (segment (start 150.26 86.36) (end 149.425 86.36) (width 0.2) (layer "F.Cu") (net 12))
 (segment (start 127.8733 120.5705) (end 127.1588 121.285) (width 0.2) (layer "F.Cu") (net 12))
 (segment (start 128.588 119.856) (end 128.588 119.062) (width 0.2) (layer "F.Cu") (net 12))
 (segment (start 127.8735 120.5705) (end 128.588 119.856) (width 0.2) (layer "F.Cu") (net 12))
 (segment (start 127.159 121.285) (end 127.8735 120.5705) (width 0.2) (layer "F.Cu") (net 12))
 (via (at 128.588 119.062) (size 0.6) (drill 0.3) (layers "F.Cu" "B.Cu") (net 12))
 (segment (start 148.362 87.423) (end 149.425 86.36) (width 0.2) (layer "B.Cu") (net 12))
 (segment (start 128.588 117.875) (end 148.362 98.1004) (width 0.2) (layer "B.Cu") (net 12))
 (segment (start 128.588 119.062) (end 128.588 117.875) (width 0.2) (layer "B.Cu") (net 12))
 (segment (start 148.362 98.1004) (end 148.362 87.423) (width 0.2) (layer "B.Cu") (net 12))
 (segment (start 145.256 85.725) (end 145.256 86.823) (width 0.2) (layer "F.Cu") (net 2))
 (segment (start 149.425 83.82) (end 147.161 83.82) (width 0.2) (layer "F.Cu") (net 2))
 (segment (start 150.26 83.82) (end 149.425 83.82) (width 0.2) (layer "F.Cu") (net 2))
 (segment (start 147.161 83.82) (end 145.256 85.725) (width 0.2) (layer "F.Cu") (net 2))
 (via (at 145.256 86.823) (size 0.6) (drill 0.3) (layers "F.Cu" "B.Cu") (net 2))
 (segment (start 146.209 105.203) (end 146.209 121.285) (width 0.2) (layer "B.Cu") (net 2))
 (segment (start 150.488 85.9197) (end 150.488 100.924) (width 0.2) (layer "B.Cu") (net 2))
 (segment (start 145.256 86.823) (end 146.782 85.297) (width 0.2) (layer "B.Cu") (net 2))
 (segment (start 146.2088 121.285) (end 146.209 121.285) (width 0.2) (layer "B.Cu") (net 2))
 (segment (start 146.782 85.297) (end 149.865 85.297) (width 0.2) (layer "B.Cu") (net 2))
 (segment (start 149.865 85.297) (end 150.488 85.9197) (width 0.2) (layer "B.Cu") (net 2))
 (segment (start 150.488 100.924) (end 146.209 105.203) (width 0.2) (layer "B.Cu") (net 2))
 (segment (start 134.185 78.74) (end 133.35 78.74) (width 0.2) (layer "F.Cu") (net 4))
 (segment (start 134.185 88.9) (end 133.35 88.9) (width 0.2) (layer "F.Cu") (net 8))
 (segment (start 133.35 91.44) (end 134.185 91.44) (width 0.2) (layer "F.Cu") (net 9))
 (segment (start 149.425 81.28) (end 150.26 81.28) (width 0.2) (layer "F.Cu") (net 13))
 (segment (start 134.185 76.2) (end 133.35 76.2) (width 0.2) (layer "F.Cu") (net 3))
 (segment (start 134.185 83.82) (end 133.35 83.82) (width 0.2) (layer "F.Cu") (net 6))
 (segment (start 133.35 81.28) (end 134.185 81.28) (width 0.2) (layer "F.Cu") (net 5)))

